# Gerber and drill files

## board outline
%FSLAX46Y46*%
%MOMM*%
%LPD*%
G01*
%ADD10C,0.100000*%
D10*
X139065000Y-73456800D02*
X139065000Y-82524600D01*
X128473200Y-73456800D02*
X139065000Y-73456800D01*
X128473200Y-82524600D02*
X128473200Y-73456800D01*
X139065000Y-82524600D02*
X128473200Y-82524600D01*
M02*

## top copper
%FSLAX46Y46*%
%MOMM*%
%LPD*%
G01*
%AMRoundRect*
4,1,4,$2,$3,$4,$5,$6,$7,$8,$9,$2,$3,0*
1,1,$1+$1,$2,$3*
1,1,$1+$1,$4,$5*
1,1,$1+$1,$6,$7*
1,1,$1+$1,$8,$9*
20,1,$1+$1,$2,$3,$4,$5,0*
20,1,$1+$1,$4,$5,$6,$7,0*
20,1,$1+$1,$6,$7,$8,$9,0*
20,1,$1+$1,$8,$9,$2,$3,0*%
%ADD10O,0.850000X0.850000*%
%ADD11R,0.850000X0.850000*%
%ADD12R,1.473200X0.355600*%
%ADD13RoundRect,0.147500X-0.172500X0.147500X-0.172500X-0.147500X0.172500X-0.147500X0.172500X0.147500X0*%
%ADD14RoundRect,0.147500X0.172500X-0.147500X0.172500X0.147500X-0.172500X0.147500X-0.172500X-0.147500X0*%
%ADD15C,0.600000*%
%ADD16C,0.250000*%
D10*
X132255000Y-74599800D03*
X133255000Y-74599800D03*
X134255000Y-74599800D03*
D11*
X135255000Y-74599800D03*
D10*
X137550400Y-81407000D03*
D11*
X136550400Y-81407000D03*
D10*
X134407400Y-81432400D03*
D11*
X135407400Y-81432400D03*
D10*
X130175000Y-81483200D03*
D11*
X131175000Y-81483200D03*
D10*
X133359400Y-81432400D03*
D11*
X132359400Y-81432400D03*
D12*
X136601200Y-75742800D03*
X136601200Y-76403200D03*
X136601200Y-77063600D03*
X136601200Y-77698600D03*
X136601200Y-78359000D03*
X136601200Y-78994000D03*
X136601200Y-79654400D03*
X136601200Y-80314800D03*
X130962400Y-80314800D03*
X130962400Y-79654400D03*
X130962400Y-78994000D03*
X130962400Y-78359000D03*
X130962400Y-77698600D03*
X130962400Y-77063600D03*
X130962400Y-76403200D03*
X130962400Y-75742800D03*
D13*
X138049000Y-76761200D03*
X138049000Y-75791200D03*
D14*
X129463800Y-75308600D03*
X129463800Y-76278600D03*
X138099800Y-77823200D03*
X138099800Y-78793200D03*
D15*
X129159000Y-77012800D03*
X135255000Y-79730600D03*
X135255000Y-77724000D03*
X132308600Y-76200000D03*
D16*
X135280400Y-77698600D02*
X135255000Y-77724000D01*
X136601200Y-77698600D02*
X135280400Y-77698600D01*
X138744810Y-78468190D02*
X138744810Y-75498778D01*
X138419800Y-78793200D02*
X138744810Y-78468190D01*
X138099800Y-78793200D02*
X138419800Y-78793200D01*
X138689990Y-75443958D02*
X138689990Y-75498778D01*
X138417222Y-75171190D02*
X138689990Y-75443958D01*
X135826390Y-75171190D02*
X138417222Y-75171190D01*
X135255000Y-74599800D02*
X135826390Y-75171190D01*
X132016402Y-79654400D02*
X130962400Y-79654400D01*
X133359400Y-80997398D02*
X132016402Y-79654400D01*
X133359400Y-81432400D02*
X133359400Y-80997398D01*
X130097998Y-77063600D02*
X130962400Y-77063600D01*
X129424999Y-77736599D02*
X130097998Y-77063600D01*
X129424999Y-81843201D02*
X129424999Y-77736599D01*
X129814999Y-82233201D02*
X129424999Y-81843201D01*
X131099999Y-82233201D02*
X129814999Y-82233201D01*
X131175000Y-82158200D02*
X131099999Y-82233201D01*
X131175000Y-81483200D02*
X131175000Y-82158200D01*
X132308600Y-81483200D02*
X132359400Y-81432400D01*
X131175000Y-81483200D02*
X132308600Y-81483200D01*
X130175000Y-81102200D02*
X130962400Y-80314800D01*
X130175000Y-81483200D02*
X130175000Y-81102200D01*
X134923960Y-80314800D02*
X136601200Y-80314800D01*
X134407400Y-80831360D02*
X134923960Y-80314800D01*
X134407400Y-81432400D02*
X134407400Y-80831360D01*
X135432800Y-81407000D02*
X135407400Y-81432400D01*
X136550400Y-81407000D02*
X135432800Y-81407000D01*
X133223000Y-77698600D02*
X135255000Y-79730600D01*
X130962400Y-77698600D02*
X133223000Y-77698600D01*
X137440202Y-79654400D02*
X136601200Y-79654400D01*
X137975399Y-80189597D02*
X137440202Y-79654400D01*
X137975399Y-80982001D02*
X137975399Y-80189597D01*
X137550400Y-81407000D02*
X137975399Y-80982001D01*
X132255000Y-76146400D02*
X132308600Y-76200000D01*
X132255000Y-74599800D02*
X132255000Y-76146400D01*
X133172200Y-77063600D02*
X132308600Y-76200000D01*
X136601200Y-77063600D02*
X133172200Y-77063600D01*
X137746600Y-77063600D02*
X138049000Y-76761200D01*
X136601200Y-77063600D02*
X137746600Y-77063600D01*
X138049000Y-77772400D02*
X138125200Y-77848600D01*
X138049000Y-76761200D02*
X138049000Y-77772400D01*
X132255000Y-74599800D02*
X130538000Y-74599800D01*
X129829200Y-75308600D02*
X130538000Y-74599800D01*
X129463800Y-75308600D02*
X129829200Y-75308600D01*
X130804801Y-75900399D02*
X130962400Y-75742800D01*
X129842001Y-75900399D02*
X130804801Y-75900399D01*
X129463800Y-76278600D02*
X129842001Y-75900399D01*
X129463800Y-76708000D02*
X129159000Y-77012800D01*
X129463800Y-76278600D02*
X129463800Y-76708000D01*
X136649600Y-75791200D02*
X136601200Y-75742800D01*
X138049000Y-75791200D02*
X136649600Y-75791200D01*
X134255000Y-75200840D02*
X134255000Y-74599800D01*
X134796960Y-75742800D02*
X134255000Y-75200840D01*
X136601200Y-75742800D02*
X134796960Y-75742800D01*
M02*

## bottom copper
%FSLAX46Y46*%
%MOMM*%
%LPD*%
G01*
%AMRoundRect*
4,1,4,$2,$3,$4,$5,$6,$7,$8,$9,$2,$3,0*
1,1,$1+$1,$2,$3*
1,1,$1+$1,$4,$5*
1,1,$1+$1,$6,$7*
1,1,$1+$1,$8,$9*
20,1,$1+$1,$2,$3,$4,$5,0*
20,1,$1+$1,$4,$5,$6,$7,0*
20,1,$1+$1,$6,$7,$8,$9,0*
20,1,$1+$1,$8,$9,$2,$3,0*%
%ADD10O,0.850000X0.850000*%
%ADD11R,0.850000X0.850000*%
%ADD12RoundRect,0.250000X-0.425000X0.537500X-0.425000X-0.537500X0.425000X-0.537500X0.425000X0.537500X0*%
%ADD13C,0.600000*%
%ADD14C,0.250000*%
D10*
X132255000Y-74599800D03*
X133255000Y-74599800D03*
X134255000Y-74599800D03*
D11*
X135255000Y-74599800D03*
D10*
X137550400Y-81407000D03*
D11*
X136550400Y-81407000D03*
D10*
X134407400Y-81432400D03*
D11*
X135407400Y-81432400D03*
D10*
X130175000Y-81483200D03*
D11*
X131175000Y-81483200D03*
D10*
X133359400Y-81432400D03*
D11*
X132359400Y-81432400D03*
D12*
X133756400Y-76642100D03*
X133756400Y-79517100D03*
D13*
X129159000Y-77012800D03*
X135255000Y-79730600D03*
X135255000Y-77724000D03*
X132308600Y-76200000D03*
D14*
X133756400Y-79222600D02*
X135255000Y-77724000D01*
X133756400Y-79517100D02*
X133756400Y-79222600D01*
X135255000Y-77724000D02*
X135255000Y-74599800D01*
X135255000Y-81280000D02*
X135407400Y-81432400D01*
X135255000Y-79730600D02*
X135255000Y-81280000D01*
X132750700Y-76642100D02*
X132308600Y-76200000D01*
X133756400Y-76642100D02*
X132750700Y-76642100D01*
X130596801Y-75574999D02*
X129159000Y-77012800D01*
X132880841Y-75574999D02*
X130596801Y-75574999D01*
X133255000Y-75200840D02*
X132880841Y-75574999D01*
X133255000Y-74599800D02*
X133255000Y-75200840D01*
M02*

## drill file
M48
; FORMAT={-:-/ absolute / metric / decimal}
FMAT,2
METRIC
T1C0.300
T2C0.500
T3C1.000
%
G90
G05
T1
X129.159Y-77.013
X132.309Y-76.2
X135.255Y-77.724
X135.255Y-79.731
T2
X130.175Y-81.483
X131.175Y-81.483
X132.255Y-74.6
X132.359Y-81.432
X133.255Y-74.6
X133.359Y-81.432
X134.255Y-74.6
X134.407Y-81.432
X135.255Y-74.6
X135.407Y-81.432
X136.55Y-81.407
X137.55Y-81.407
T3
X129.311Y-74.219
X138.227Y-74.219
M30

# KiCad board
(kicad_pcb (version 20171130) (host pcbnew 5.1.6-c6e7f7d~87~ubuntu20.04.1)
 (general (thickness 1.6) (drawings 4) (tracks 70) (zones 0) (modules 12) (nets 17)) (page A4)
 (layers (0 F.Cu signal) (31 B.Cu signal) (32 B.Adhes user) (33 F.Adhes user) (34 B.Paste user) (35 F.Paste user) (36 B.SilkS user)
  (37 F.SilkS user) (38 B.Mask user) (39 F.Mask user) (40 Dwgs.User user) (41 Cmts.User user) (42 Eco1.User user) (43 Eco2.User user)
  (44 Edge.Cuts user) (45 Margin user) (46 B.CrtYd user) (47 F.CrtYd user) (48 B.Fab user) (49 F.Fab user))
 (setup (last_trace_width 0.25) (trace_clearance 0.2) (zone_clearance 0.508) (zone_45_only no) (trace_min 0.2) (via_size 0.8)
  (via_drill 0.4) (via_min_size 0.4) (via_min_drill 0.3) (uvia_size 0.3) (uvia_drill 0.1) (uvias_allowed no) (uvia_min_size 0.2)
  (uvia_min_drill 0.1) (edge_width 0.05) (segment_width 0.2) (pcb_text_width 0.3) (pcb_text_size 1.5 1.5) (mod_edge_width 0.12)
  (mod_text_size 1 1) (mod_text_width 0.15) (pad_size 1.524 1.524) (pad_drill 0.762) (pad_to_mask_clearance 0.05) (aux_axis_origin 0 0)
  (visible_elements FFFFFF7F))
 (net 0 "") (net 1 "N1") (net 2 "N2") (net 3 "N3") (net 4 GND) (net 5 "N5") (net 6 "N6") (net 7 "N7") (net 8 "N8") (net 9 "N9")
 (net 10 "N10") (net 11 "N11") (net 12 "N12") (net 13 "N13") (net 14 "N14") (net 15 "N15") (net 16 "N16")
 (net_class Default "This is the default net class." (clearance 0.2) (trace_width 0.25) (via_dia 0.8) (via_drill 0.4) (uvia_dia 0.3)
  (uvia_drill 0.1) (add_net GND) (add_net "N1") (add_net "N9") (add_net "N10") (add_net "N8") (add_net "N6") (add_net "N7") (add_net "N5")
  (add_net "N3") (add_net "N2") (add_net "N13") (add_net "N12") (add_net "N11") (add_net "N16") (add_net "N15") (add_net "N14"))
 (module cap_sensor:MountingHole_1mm (layer F.Cu) (at 138.2268 74.2188)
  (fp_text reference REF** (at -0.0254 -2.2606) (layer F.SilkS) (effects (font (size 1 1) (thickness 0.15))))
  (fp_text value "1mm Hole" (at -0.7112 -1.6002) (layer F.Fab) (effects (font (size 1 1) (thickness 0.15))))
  (pad "" np_thru_hole circle (at 0 0) (size 1 1) (drill 1) (layers *.Cu *.Mask)))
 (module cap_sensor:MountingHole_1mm (layer F.Cu) (at 129.3114 74.2188)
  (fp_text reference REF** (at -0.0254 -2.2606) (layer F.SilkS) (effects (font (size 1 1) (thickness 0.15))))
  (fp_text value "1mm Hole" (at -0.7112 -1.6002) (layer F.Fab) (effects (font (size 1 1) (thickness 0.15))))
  (pad "" np_thru_hole circle (at 0 0) (size 1 1) (drill 1) (layers *.Cu *.Mask)))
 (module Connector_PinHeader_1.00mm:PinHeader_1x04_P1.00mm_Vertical (layer F.Cu) (at 135.255 74.5998 270)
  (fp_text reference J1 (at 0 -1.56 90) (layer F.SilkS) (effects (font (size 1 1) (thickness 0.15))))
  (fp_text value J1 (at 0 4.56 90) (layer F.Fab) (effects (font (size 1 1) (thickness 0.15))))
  (pad 4 thru_hole oval (at 0 3 270) (size 0.85 0.85) (drill 0.5) (layers *.Cu *.Mask) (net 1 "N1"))
  (pad 3 thru_hole oval (at 0 2 270) (size 0.85 0.85) (drill 0.5) (layers *.Cu *.Mask) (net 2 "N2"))
  (pad 2 thru_hole oval (at 0 1 270) (size 0.85 0.85) (drill 0.5) (layers *.Cu *.Mask) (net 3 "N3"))
  (pad 1 thru_hole rect (at 0 0 270) (size 0.85 0.85) (drill 0.5) (layers *.Cu *.Mask) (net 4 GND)))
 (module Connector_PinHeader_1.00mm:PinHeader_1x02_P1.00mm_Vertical (layer F.Cu) (at 136.5504 81.407 90)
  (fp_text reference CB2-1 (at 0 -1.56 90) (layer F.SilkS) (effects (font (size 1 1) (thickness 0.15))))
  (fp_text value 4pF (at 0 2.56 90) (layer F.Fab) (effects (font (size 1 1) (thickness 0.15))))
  (pad 2 thru_hole oval (at 0 1 90) (size 0.85 0.85) (drill 0.5) (layers *.Cu *.Mask) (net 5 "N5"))
  (pad 1 thru_hole rect (at 0 0 90) (size 0.85 0.85) (drill 0.5) (layers *.Cu *.Mask) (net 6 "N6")))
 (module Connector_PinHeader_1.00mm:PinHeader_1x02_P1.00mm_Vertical (layer F.Cu) (at 135.4074 81.4324 270)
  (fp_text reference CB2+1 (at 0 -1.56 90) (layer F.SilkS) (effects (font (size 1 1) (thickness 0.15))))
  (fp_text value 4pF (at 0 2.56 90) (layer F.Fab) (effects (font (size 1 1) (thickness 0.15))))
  (pad 2 thru_hole oval (at 0 1 270) (size 0.85 0.85) (drill 0.5) (layers *.Cu *.Mask) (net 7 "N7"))
  (pad 1 thru_hole rect (at 0 0 270) (size 0.85 0.85) (drill 0.5) (layers *.Cu *.Mask) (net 6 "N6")))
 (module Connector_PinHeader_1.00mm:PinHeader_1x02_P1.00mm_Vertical (layer F.Cu) (at 131.175 81.4832 270)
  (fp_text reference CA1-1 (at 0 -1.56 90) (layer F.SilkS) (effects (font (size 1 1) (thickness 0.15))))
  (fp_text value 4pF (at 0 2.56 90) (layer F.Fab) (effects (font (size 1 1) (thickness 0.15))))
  (pad 2 thru_hole oval (at 0 1 270) (size 0.85 0.85) (drill 0.5) (layers *.Cu *.Mask) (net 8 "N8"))
  (pad 1 thru_hole rect (at 0 0 270) (size 0.85 0.85) (drill 0.5) (layers *.Cu *.Mask) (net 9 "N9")))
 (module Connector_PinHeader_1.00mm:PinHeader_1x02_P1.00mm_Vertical (layer F.Cu) (at 132.3594 81.4324 90)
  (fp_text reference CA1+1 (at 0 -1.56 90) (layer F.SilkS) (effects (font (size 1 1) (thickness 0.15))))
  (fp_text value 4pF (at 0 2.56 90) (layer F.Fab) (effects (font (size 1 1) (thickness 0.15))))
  (pad 2 thru_hole oval (at 0 1 90) (size 0.85 0.85) (drill 0.5) (layers *.Cu *.Mask) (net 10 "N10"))
  (pad 1 thru_hole rect (at 0 0 90) (size 0.85 0.85) (drill 0.5) (layers *.Cu *.Mask) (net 9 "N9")))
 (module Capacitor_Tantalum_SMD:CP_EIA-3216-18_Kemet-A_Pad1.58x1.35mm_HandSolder (layer B.Cu) (at 133.7564 78.0796 270)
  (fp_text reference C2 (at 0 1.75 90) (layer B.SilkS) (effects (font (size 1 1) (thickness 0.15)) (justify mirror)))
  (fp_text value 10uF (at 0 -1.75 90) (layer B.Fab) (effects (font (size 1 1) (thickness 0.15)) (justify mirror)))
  (pad 1 smd roundrect (at -1.4375 0 270) (size 1.575 1.35) (layers B.Cu B.Paste B.Mask) (roundrect_rratio 0.185185) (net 1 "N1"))
  (pad 2 smd roundrect (at 1.4375 0 270) (size 1.575 1.35) (layers B.Cu B.Paste B.Mask) (roundrect_rratio 0.185185) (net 4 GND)))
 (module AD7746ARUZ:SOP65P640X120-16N (layer F.Cu) (at 133.7818 78.0288)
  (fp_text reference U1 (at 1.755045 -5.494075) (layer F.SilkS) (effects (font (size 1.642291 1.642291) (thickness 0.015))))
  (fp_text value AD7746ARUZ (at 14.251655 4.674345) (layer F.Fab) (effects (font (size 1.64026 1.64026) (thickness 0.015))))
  (pad 16 smd rect (at 2.8194 -2.286) (size 1.4732 0.3556) (layers F.Cu F.Paste F.Mask) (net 3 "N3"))
  (pad 15 smd rect (at 2.8194 -1.6256) (size 1.4732 0.3556) (layers F.Cu F.Paste F.Mask) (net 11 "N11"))
  (pad 14 smd rect (at 2.8194 -0.9652) (size 1.4732 0.3556) (layers F.Cu F.Paste F.Mask) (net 1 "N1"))
  (pad 13 smd rect (at 2.8194 -0.3302) (size 1.4732 0.3556) (layers F.Cu F.Paste F.Mask) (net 4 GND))
  (pad 12 smd rect (at 2.8194 0.3302) (size 1.4732 0.3556) (layers F.Cu F.Paste F.Mask) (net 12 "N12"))
  (pad 11 smd rect (at 2.8194 0.9652) (size 1.4732 0.3556) (layers F.Cu F.Paste F.Mask) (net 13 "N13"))
  (pad 10 smd rect (at 2.8194 1.6256) (size 1.4732 0.3556) (layers F.Cu F.Paste F.Mask) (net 5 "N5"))
  (pad 9 smd rect (at 2.8194 2.286) (size 1.4732 0.3556) (layers F.Cu F.Paste F.Mask) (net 7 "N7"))
  (pad 8 smd rect (at -2.8194 2.286) (size 1.4732 0.3556) (layers F.Cu F.Paste F.Mask) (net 8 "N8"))
  (pad 7 smd rect (at -2.8194 1.6256) (size 1.4732 0.3556) (layers F.Cu F.Paste F.Mask) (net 10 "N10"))
  (pad 6 smd rect (at -2.8194 0.9652) (size 1.4732 0.3556) (layers F.Cu F.Paste F.Mask) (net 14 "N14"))
  (pad 5 smd rect (at -2.8194 0.3302) (size 1.4732 0.3556) (layers F.Cu F.Paste F.Mask) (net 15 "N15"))
  (pad 4 smd rect (at -2.8194 -0.3302) (size 1.4732 0.3556) (layers F.Cu F.Paste F.Mask) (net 6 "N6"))
  (pad 3 smd rect (at -2.8194 -0.9652) (size 1.4732 0.3556) (layers F.Cu F.Paste F.Mask) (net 9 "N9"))
  (pad 2 smd rect (at -2.8194 -1.6256) (size 1.4732 0.3556) (layers F.Cu F.Paste F.Mask) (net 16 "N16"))
  (pad 1 smd rect (at -2.8194 -2.286) (size 1.4732 0.3556) (layers F.Cu F.Paste F.Mask) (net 2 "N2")))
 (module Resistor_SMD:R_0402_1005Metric (layer F.Cu) (at 138.049 76.2762 270)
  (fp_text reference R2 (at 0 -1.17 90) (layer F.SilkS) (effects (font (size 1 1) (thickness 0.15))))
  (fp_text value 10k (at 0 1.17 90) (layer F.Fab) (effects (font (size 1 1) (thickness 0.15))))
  (pad 2 smd roundrect (at 0.485 0 270) (size 0.59 0.64) (layers F.Cu F.Paste F.Mask) (roundrect_rratio 0.25) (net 1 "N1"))
  (pad 1 smd roundrect (at -0.485 0 270) (size 0.59 0.64) (layers F.Cu F.Paste F.Mask) (roundrect_rratio 0.25) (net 3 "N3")))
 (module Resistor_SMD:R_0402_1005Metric (layer F.Cu) (at 129.4638 75.7936 90)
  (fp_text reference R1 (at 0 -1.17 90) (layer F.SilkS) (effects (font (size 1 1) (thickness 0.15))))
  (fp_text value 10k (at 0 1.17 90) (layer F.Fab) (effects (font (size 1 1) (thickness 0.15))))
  (pad 2 smd roundrect (at 0.485 0 90) (size 0.59 0.64) (layers F.Cu F.Paste F.Mask) (roundrect_rratio 0.25) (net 1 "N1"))
  (pad 1 smd roundrect (at -0.485 0 90) (size 0.59 0.64) (layers F.Cu F.Paste F.Mask) (roundrect_rratio 0.25) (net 2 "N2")))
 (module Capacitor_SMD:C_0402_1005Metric (layer F.Cu) (at 138.0998 78.3082 90)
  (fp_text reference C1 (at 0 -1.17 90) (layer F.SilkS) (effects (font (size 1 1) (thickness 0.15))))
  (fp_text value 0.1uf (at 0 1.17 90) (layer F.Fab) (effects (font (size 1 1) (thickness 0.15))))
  (pad 2 smd roundrect (at 0.485 0 90) (size 0.59 0.64) (layers F.Cu F.Paste F.Mask) (roundrect_rratio 0.25) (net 1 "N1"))
  (pad 1 smd roundrect (at -0.485 0 90) (size 0.59 0.64) (layers F.Cu F.Paste F.Mask) (roundrect_rratio 0.25) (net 4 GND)))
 (gr_line (start 139.065 73.4568) (end 139.065 82.5246) (layer Edge.Cuts) (width 0.1))
 (gr_line (start 128.4732 73.4568) (end 139.065 73.4568) (layer Edge.Cuts) (width 0.1))
 (gr_line (start 128.4732 82.5246) (end 128.4732 73.4568) (layer Edge.Cuts) (width 0.1))
 (gr_line (start 139.065 82.5246) (end 128.4732 82.5246) (layer Edge.Cuts) (width 0.1))
 (via (at 129.159 77.0128) (size 0.6) (drill 0.3) (layers F.Cu B.Cu) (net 2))
 (via (at 135.255 79.7306) (size 0.6) (drill 0.3) (layers F.Cu B.Cu) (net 6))
 (via (at 135.255 77.724) (size 0.6) (drill 0.3) (layers F.Cu B.Cu) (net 4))
 (segment (start 133.7564 79.2226) (end 135.255 77.724) (width 0.25) (layer B.Cu) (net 4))
 (segment (start 133.7564 79.5171) (end 133.7564 79.2226) (width 0.25) (layer B.Cu) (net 4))
 (segment (start 135.2804 77.6986) (end 135.255 77.724) (width 0.25) (layer F.Cu) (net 4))
 (segment (start 136.6012 77.6986) (end 135.2804 77.6986) (width 0.25) (layer F.Cu) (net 4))
 (segment (start 135.255 77.724) (end 135.255 74.5998) (width 0.25) (layer B.Cu) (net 4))
 (segment (start 138.74481 78.46819) (end 138.74481 75.498778) (width 0.25) (layer F.Cu) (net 4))
 (segment (start 138.4198 78.7932) (end 138.74481 78.46819) (width 0.25) (layer F.Cu) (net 4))
 (segment (start 138.0998 78.7932) (end 138.4198 78.7932) (width 0.25) (layer F.Cu) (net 4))
 (segment (start 138.68999 75.443958) (end 138.68999 75.498778) (width 0.25) (layer F.Cu) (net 4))
 (segment (start 138.417222 75.17119) (end 138.68999 75.443958) (width 0.25) (layer F.Cu) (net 4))
 (segment (start 135.82639 75.17119) (end 138.417222 75.17119) (width 0.25) (layer F.Cu) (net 4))
 (segment (start 135.255 74.5998) (end 135.82639 75.17119) (width 0.25) (layer F.Cu) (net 4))
 (segment (start 132.016402 79.6544) (end 130.9624 79.6544) (width 0.25) (layer F.Cu) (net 10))
 (segment (start 133.3594 80.997398) (end 132.016402 79.6544) (width 0.25) (layer F.Cu) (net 10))
 (segment (start 133.3594 81.4324) (end 133.3594 80.997398) (width 0.25) (layer F.Cu) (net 10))
 (segment (start 130.097998 77.0636) (end 130.9624 77.0636) (width 0.25) (layer F.Cu) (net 9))
 (segment (start 129.424999 77.736599) (end 130.097998 77.0636) (width 0.25) (layer F.Cu) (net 9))
 (segment (start 129.424999 81.843201) (end 129.424999 77.736599) (width 0.25) (layer F.Cu) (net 9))
 (segment (start 129.814999 82.233201) (end 129.424999 81.843201) (width 0.25) (layer F.Cu) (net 9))
 (segment (start 131.099999 82.233201) (end 129.814999 82.233201) (width 0.25) (layer F.Cu) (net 9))
 (segment (start 131.175 82.1582) (end 131.099999 82.233201) (width 0.25) (layer F.Cu) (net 9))
 (segment (start 131.175 81.4832) (end 131.175 82.1582) (width 0.25) (layer F.Cu) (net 9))
 (segment (start 132.3086 81.4832) (end 132.3594 81.4324) (width 0.25) (layer F.Cu) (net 9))
 (segment (start 131.175 81.4832) (end 132.3086 81.4832) (width 0.25) (layer F.Cu) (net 9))
 (segment (start 130.175 81.1022) (end 130.9624 80.3148) (width 0.25) (layer F.Cu) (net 8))
 (segment (start 130.175 81.4832) (end 130.175 81.1022) (width 0.25) (layer F.Cu) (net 8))
 (segment (start 134.92396 80.3148) (end 136.6012 80.3148) (width 0.25) (layer F.Cu) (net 7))
 (segment (start 134.4074 80.83136) (end 134.92396 80.3148) (width 0.25) (layer F.Cu) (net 7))
 (segment (start 134.4074 81.4324) (end 134.4074 80.83136) (width 0.25) (layer F.Cu) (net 7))
 (segment (start 135.4328 81.407) (end 135.4074 81.4324) (width 0.25) (layer F.Cu) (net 6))
 (segment (start 136.5504 81.407) (end 135.4328 81.407) (width 0.25) (layer F.Cu) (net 6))
 (segment (start 135.255 81.28) (end 135.4074 81.4324) (width 0.25) (layer B.Cu) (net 6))
 (segment (start 135.255 79.7306) (end 135.255 81.28) (width 0.25) (layer B.Cu) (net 6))
 (segment (start 133.223 77.6986) (end 135.255 79.7306) (width 0.25) (layer F.Cu) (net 6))
 (segment (start 130.9624 77.6986) (end 133.223 77.6986) (width 0.25) (layer F.Cu) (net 6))
 (segment (start 137.440202 79.6544) (end 136.6012 79.6544) (width 0.25) (layer F.Cu) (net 5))
 (segment (start 137.975399 80.189597) (end 137.440202 79.6544) (width 0.25) (layer F.Cu) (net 5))
 (segment (start 137.975399 80.982001) (end 137.975399 80.189597) (width 0.25) (layer F.Cu) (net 5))
 (segment (start 137.5504 81.407) (end 137.975399 80.982001) (width 0.25) (layer F.Cu) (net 5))
 (via (at 132.3086 76.2) (size 0.6) (drill 0.3) (layers F.Cu B.Cu) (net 1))
 (segment (start 132.255 76.1464) (end 132.3086 76.2) (width 0.25) (layer F.Cu) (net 1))
 (segment (start 132.255 74.5998) (end 132.255 76.1464) (width 0.25) (layer F.Cu) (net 1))
 (segment (start 132.7507 76.6421) (end 132.3086 76.2) (width 0.25) (layer B.Cu) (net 1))
 (segment (start 133.7564 76.6421) (end 132.7507 76.6421) (width 0.25) (layer B.Cu) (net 1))
 (segment (start 133.1722 77.0636) (end 132.3086 76.2) (width 0.25) (layer F.Cu) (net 1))
 (segment (start 136.6012 77.0636) (end 133.1722 77.0636) (width 0.25) (layer F.Cu) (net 1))
 (segment (start 137.7466 77.0636) (end 138.049 76.7612) (width 0.25) (layer F.Cu) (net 1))
 (segment (start 136.6012 77.0636) (end 137.7466 77.0636) (width 0.25) (layer F.Cu) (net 1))
 (segment (start 138.049 77.7724) (end 138.1252 77.8486) (width 0.25) (layer F.Cu) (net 1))
 (segment (start 138.049 76.7612) (end 138.049 77.7724) (width 0.25) (layer F.Cu) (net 1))
 (segment (start 132.255 74.5998) (end 130.538 74.5998) (width 0.25) (layer F.Cu) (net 1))
 (segment (start 129.8292 75.3086) (end 130.538 74.5998) (width 0.25) (layer F.Cu) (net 1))
 (segment (start 129.4638 75.3086) (end 129.8292 75.3086) (width 0.25) (layer F.Cu) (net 1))
 (segment (start 130.804801 75.900399) (end 130.9624 75.7428) (width 0.25) (layer F.Cu) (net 2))
 (segment (start 129.842001 75.900399) (end 130.804801 75.900399) (width 0.25) (layer F.Cu) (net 2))
 (segment (start 129.4638 76.2786) (end 129.842001 75.900399) (width 0.25) (layer F.Cu) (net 2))
 (segment (start 130.596801 75.574999) (end 129.159 77.0128) (width 0.25) (layer B.Cu) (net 2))
 (segment (start 132.880841 75.574999) (end 130.596801 75.574999) (width 0.25) (layer B.Cu) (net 2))
 (segment (start 133.255 75.20084) (end 132.880841 75.574999) (width 0.25) (layer B.Cu) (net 2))
 (segment (start 133.255 74.5998) (end 133.255 75.20084) (width 0.25) (layer B.Cu) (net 2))
 (segment (start 129.4638 76.708) (end 129.159 77.0128) (width 0.25) (layer F.Cu) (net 2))
 (segment (start 129.4638 76.2786) (end 129.4638 76.708) (width 0.25) (layer F.Cu) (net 2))
 (segment (start 136.6496 75.7912) (end 136.6012 75.7428) (width 0.25) (layer F.Cu) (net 3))
 (segment (start 138.049 75.7912) (end 136.6496 75.7912) (width 0.25) (layer F.Cu) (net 3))
 (segment (start 134.255 75.20084) (end 134.255 74.5998) (width 0.25) (layer F.Cu) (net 3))
 (segment (start 134.79696 75.7428) (end 134.255 75.20084) (width 0.25) (layer F.Cu) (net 3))
 (segment (start 136.6012 75.7428) (end 134.79696 75.7428) (width 0.25) (layer F.Cu) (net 3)))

